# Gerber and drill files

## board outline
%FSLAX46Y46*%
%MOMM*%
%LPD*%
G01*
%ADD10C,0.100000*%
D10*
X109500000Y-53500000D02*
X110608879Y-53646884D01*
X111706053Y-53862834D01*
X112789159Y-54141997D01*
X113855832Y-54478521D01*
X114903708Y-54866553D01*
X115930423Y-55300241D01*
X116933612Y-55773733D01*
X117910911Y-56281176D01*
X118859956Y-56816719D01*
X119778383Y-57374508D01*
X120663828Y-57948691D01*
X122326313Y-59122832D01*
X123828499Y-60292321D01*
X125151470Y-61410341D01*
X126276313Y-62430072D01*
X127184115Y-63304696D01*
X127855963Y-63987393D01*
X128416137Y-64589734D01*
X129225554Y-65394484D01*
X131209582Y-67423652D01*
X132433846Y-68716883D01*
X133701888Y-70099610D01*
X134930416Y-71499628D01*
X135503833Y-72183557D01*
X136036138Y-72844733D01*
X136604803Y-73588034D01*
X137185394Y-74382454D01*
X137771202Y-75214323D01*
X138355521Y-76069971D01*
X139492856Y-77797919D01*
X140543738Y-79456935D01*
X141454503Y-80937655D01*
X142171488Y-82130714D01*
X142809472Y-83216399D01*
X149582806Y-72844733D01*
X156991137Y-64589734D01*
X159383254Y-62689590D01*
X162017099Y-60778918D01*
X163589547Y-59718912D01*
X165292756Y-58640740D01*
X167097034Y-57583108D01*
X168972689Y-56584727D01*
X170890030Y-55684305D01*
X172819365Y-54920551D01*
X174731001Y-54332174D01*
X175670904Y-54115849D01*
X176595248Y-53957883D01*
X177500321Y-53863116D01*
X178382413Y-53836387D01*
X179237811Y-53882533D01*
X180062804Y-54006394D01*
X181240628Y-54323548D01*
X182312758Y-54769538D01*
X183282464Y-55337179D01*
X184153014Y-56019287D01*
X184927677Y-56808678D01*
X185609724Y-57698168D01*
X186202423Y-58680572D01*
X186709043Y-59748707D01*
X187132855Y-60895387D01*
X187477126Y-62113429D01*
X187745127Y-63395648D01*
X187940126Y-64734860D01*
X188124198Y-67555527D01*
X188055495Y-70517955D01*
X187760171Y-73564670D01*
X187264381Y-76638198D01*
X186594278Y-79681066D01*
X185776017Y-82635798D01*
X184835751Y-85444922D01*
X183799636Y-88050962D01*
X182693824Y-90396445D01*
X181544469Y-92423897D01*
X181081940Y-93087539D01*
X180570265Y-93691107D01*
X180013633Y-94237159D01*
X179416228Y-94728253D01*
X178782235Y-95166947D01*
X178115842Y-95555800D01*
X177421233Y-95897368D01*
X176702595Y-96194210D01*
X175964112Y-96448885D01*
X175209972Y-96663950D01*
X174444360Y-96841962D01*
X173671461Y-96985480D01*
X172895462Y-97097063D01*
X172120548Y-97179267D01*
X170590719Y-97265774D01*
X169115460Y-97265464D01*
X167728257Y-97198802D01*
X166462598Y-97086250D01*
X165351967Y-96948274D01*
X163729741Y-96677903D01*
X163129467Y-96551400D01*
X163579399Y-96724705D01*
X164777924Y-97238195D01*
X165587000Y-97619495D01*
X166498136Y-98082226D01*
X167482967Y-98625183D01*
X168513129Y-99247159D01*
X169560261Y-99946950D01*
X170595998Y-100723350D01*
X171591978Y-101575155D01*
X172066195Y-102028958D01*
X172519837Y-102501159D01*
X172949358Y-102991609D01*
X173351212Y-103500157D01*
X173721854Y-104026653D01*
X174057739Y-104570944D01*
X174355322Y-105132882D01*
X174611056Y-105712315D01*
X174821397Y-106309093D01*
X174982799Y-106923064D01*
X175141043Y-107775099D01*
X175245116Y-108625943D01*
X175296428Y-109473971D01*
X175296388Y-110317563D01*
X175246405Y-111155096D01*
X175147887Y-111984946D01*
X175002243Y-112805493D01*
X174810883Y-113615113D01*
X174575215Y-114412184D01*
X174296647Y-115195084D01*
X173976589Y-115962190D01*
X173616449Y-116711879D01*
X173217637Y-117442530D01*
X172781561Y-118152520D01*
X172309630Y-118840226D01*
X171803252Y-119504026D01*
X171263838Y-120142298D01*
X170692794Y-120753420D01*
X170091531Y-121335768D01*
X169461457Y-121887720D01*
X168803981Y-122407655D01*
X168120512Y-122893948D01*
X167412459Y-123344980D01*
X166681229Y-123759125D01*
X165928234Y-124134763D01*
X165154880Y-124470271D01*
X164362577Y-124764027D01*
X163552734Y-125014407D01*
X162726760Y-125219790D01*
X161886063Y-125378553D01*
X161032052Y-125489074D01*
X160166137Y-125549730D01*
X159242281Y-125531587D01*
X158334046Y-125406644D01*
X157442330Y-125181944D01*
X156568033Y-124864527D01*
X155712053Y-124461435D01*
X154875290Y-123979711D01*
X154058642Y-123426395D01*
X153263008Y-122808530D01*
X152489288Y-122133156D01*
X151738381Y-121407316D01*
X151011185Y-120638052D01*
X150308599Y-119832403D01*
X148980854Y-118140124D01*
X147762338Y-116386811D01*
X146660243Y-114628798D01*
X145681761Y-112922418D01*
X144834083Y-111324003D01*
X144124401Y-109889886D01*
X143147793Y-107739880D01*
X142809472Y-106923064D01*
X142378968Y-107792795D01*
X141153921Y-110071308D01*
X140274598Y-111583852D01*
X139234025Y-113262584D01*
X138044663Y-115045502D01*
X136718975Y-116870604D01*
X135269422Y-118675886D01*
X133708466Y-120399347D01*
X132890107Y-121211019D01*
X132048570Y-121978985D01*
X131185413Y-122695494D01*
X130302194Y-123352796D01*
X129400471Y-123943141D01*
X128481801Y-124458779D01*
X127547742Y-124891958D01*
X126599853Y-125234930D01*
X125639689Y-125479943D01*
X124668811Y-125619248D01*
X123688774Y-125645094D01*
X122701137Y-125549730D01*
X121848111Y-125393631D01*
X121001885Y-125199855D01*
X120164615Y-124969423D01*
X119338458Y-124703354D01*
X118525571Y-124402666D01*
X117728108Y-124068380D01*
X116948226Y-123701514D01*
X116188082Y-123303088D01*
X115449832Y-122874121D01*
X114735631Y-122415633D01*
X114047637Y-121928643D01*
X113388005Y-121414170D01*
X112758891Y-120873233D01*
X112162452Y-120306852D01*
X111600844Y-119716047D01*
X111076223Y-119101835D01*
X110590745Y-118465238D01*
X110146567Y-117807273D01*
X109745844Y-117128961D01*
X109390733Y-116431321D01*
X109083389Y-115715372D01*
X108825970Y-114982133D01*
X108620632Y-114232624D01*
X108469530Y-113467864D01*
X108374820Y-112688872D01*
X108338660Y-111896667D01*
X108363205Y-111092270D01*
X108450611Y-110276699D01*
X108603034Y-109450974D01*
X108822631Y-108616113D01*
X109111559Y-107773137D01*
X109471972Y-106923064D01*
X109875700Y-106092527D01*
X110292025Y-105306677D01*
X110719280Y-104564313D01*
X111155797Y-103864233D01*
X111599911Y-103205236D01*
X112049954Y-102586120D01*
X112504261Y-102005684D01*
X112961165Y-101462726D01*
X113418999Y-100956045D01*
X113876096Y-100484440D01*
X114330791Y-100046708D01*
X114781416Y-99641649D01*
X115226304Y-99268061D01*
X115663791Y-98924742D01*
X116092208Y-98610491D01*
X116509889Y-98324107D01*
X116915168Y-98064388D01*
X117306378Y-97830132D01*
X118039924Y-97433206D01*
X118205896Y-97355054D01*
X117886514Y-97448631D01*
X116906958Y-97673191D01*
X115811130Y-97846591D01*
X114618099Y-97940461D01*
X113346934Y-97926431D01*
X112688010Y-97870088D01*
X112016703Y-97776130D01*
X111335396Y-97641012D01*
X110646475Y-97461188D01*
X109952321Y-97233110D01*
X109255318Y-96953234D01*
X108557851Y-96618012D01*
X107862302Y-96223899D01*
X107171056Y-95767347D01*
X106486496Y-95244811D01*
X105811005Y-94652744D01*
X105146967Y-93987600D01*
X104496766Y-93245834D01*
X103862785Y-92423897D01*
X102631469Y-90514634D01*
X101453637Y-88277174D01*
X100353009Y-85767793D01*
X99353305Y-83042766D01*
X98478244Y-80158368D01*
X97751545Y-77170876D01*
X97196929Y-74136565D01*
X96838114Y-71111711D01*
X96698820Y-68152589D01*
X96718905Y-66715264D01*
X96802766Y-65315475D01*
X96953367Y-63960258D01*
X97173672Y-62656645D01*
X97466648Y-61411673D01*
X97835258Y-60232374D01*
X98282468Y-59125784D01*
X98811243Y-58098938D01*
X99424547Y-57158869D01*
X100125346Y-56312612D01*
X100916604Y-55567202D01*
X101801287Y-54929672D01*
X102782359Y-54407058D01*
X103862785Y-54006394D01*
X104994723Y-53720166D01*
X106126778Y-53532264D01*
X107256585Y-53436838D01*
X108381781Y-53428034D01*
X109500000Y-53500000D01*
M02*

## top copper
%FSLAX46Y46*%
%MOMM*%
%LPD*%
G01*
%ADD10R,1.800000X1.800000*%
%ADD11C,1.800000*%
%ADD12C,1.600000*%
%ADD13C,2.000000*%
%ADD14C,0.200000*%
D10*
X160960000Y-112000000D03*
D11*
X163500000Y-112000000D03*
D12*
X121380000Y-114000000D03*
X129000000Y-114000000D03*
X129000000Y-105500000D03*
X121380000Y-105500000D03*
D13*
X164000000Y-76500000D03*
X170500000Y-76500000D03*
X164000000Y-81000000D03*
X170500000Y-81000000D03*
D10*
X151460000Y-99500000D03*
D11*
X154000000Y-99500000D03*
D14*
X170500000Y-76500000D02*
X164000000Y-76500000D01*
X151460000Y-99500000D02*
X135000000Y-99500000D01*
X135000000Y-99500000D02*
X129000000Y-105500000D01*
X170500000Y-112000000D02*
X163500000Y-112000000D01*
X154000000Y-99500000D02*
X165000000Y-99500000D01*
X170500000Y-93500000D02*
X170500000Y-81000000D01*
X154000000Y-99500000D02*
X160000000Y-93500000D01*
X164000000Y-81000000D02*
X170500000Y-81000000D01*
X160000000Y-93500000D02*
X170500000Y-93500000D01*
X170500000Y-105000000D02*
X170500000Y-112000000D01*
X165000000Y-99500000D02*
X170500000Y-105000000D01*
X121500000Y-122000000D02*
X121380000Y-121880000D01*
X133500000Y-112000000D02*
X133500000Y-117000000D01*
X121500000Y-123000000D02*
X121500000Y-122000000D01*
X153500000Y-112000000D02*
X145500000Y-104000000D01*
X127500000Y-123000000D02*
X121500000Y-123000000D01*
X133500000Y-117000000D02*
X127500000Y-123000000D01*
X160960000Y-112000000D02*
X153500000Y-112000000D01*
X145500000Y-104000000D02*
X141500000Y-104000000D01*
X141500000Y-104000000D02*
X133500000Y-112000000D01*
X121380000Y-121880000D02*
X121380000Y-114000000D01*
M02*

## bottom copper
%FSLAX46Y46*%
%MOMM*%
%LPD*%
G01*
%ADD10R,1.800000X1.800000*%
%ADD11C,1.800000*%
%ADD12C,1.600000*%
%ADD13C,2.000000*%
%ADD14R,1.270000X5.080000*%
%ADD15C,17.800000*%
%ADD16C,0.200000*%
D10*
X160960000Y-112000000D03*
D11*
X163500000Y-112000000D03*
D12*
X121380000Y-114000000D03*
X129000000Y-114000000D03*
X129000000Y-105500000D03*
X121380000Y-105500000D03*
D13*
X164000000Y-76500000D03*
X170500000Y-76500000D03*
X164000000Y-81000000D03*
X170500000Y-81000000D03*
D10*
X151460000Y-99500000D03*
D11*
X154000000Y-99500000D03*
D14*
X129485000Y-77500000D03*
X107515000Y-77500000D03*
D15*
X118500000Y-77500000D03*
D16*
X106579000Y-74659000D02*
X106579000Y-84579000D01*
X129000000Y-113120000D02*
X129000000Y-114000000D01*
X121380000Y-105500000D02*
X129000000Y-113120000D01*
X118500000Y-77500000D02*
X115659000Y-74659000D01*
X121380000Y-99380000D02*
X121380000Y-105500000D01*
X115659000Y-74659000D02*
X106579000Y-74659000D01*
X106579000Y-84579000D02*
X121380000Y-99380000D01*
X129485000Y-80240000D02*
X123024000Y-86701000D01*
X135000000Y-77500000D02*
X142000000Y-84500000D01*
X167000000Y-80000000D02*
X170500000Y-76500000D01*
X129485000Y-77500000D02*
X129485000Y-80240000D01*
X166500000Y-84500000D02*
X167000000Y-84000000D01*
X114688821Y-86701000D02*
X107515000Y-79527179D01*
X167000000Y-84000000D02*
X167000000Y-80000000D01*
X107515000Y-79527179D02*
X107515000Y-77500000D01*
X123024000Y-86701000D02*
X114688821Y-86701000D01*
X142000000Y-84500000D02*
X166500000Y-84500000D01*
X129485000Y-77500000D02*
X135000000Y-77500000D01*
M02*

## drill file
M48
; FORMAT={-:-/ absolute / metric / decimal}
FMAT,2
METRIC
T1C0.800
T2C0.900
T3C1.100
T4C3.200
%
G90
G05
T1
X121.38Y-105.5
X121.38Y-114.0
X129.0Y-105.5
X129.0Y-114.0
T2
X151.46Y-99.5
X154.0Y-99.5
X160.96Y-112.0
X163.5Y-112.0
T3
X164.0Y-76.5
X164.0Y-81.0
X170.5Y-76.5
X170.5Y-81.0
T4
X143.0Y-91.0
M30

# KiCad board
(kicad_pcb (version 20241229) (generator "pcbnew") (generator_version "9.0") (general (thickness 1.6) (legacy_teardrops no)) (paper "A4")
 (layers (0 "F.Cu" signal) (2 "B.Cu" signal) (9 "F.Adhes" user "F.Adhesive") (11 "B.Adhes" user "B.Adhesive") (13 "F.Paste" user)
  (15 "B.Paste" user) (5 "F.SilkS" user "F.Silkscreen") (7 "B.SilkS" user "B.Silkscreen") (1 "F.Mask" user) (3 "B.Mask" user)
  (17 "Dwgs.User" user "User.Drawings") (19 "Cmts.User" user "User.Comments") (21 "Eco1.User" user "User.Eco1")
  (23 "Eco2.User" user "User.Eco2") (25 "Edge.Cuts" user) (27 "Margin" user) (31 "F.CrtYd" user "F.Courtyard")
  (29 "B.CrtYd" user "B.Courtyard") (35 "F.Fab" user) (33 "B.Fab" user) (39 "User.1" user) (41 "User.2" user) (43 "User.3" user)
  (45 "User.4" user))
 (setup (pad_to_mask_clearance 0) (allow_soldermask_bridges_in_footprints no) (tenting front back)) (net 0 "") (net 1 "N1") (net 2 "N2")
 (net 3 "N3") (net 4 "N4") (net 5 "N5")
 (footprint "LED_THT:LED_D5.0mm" (layer "F.Cu") (at 160.96 112)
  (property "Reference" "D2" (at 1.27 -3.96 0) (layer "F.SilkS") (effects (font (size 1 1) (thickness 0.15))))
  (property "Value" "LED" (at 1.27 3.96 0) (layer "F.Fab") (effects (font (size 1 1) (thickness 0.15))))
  (pad "1" thru_hole rect (at 0 0) (size 1.8 1.8) (drill 0.9) (layers "*.Cu" "*.Mask") (remove_unused_layers no) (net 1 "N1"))
  (pad "2" thru_hole circle (at 2.54 0) (size 1.8 1.8) (drill 0.9) (layers "*.Cu" "*.Mask") (remove_unused_layers no) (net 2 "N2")))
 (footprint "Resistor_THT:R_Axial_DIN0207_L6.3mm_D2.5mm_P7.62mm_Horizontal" (layer "F.Cu") (at 121.38 114)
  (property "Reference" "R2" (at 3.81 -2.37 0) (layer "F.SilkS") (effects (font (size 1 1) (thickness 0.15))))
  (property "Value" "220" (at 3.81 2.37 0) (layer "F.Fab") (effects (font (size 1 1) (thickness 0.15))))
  (pad "1" thru_hole circle (at 0 0) (size 1.6 1.6) (drill 0.8) (layers "*.Cu" "*.Mask") (remove_unused_layers no) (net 1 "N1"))
  (pad "2" thru_hole circle (at 7.62 0) (size 1.6 1.6) (drill 0.8) (layers "*.Cu" "*.Mask") (remove_unused_layers no) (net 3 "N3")))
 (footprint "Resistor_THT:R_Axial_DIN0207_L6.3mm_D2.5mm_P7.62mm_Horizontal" (layer "F.Cu") (at 129 105.5 180)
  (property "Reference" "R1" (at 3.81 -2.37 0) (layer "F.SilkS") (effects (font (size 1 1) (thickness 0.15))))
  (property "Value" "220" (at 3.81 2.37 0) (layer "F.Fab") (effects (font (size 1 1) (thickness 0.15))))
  (pad "1" thru_hole circle (at 0 0 180) (size 1.6 1.6) (drill 0.8) (layers "*.Cu" "*.Mask") (remove_unused_layers no) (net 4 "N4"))
  (pad "2" thru_hole circle (at 7.62 0 180) (size 1.6 1.6) (drill 0.8) (layers "*.Cu" "*.Mask") (remove_unused_layers no) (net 3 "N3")))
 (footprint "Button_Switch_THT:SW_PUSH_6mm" (layer "F.Cu") (at 164 76.5)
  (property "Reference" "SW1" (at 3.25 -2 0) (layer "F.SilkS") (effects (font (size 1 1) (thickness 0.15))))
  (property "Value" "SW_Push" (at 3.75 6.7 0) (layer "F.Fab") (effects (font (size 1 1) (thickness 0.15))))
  (pad "1" thru_hole circle (at 0 0 90) (size 2 2) (drill 1.1) (layers "*.Cu" "*.Mask") (remove_unused_layers no) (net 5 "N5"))
  (pad "1" thru_hole circle (at 6.5 0 90) (size 2 2) (drill 1.1) (layers "*.Cu" "*.Mask") (remove_unused_layers no) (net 5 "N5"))
  (pad "2" thru_hole circle (at 0 4.5 90) (size 2 2) (drill 1.1) (layers "*.Cu" "*.Mask") (remove_unused_layers no) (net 2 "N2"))
  (pad "2" thru_hole circle (at 6.5 4.5 90) (size 2 2) (drill 1.1) (layers "*.Cu" "*.Mask") (remove_unused_layers no) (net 2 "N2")))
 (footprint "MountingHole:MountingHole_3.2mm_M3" (layer "F.Cu") (at 143 91)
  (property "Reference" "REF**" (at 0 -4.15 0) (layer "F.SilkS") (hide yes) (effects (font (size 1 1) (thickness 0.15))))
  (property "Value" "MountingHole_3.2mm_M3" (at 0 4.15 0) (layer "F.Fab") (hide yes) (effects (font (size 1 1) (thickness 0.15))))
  (pad "" np_thru_hole circle (at 0 0) (size 3.2 3.2) (drill 3.2) (layers "*.Cu" "*.Mask")))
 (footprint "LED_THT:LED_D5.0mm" (layer "F.Cu") (at 151.46 99.5)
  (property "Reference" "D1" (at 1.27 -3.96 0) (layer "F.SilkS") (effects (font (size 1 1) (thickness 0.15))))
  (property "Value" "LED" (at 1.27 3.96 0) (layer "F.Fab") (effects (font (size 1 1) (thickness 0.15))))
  (pad "1" thru_hole rect (at 0 0) (size 1.8 1.8) (drill 0.9) (layers "*.Cu" "*.Mask") (remove_unused_layers no) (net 4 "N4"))
  (pad "2" thru_hole circle (at 2.54 0) (size 1.8 1.8) (drill 0.9) (layers "*.Cu" "*.Mask") (remove_unused_layers no) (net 2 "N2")))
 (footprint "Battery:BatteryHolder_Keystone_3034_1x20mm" (layer "B.Cu") (at 118.5 77.5 180)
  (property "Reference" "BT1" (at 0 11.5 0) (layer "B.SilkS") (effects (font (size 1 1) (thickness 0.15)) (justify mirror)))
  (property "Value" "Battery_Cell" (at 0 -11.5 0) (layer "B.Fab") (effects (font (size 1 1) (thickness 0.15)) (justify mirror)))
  (pad "1" smd rect (at -10.985 0 180) (size 1.27 5.08) (layers "B.Cu" "B.Mask" "B.Paste") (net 5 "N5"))
  (pad "1" smd rect (at 10.985 0 180) (size 1.27 5.08) (layers "B.Cu" "B.Mask" "B.Paste") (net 5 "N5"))
  (pad "2" smd circle (at 0 0 180) (size 17.8 17.8) (layers "B.Cu" "B.Mask") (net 3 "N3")))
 (gr_poly
  (pts (xy 109.5 53.5) (xy 110.608879 53.646884) (xy 111.706053 53.862834) (xy 112.789159 54.141997) (xy 113.855832 54.478521)
   (xy 114.903708 54.866553) (xy 115.930423 55.300241) (xy 116.933612 55.773733) (xy 117.910911 56.281176) (xy 118.859956 56.816719)
   (xy 119.778383 57.374508) (xy 120.663828 57.948691) (xy 122.326313 59.122832) (xy 123.828499 60.292321) (xy 125.15147 61.410341)
   (xy 126.276313 62.430072) (xy 127.184115 63.304696) (xy 127.855963 63.987393) (xy 128.416137 64.589734) (xy 129.225554 65.394484)
   (xy 131.209582 67.423652) (xy 132.433846 68.716883) (xy 133.701888 70.09961) (xy 134.930416 71.499628) (xy 135.503833 72.183557)
   (xy 136.036138 72.844733) (xy 136.604803 73.588034) (xy 137.185394 74.382454) (xy 137.771202 75.214323) (xy 138.355521 76.069971)
   (xy 139.492856 77.797919) (xy 140.543738 79.456935) (xy 141.454503 80.937655) (xy 142.171488 82.130714) (xy 142.809472 83.216399)
   (xy 149.582806 72.844733) (xy 156.991137 64.589734) (xy 159.383254 62.68959) (xy 162.017099 60.778918) (xy 163.589547 59.718912)
   (xy 165.292756 58.64074) (xy 167.097034 57.583108) (xy 168.972689 56.584727) (xy 170.89003 55.684305) (xy 172.819365 54.920551)
   (xy 174.731001 54.332174) (xy 175.670904 54.115849) (xy 176.595248 53.957883) (xy 177.500321 53.863116) (xy 178.382413 53.836387)
   (xy 179.237811 53.882533) (xy 180.062804 54.006394) (xy 181.240628 54.323548) (xy 182.312758 54.769538) (xy 183.282464 55.337179)
   (xy 184.153014 56.019287) (xy 184.927677 56.808678) (xy 185.609724 57.698168) (xy 186.202423 58.680572) (xy 186.709043 59.748707)
   (xy 187.132855 60.895387) (xy 187.477126 62.113429) (xy 187.745127 63.395648) (xy 187.940126 64.73486) (xy 188.124198 67.555527)
   (xy 188.055495 70.517955) (xy 187.760171 73.56467) (xy 187.264381 76.638198) (xy 186.594278 79.681066) (xy 185.776017 82.635798)
   (xy 184.835751 85.444922) (xy 183.799636 88.050962) (xy 182.693824 90.396445) (xy 181.544469 92.423897) (xy 181.08194 93.087539)
   (xy 180.570265 93.691107) (xy 180.013633 94.237159) (xy 179.416228 94.728253) (xy 178.782235 95.166947) (xy 178.115842 95.5558)
   (xy 177.421233 95.897368) (xy 176.702595 96.19421) (xy 175.964112 96.448885) (xy 175.209972 96.66395) (xy 174.44436 96.841962)
   (xy 173.671461 96.98548) (xy 172.895462 97.097063) (xy 172.120548 97.179267) (xy 170.590719 97.265774) (xy 169.11546 97.265464)
   (xy 167.728257 97.198802) (xy 166.462598 97.08625) (xy 165.351967 96.948274) (xy 163.729741 96.677903) (xy 163.129467 96.5514)
   (xy 163.579399 96.724705) (xy 164.777924 97.238195) (xy 165.587 97.619495) (xy 166.498136 98.082226) (xy 167.482967 98.625183)
   (xy 168.513129 99.247159) (xy 169.560261 99.94695) (xy 170.595998 100.72335) (xy 171.591978 101.575155) (xy 172.066195 102.028958)
   (xy 172.519837 102.501159) (xy 172.949358 102.991609) (xy 173.351212 103.500157) (xy 173.721854 104.026653) (xy 174.057739 104.570944)
   (xy 174.355322 105.132882) (xy 174.611056 105.712315) (xy 174.821397 106.309093) (xy 174.982799 106.923064) (xy 175.141043 107.775099)
   (xy 175.245116 108.625943) (xy 175.296428 109.473971) (xy 175.296388 110.317563) (xy 175.246405 111.155096) (xy 175.147887 111.984946)
   (xy 175.002243 112.805493) (xy 174.810883 113.615113) (xy 174.575215 114.412184) (xy 174.296647 115.195084) (xy 173.976589 115.96219)
   (xy 173.616449 116.711879) (xy 173.217637 117.44253) (xy 172.781561 118.15252) (xy 172.30963 118.840226) (xy 171.803252 119.504026)
   (xy 171.263838 120.142298) (xy 170.692794 120.75342) (xy 170.091531 121.335768) (xy 169.461457 121.88772) (xy 168.803981 122.407655)
   (xy 168.120512 122.893948) (xy 167.412459 123.34498) (xy 166.681229 123.759125) (xy 165.928234 124.134763) (xy 165.15488 124.470271)
   (xy 164.362577 124.764027) (xy 163.552734 125.014407) (xy 162.72676 125.21979) (xy 161.886063 125.378553) (xy 161.032052 125.489074)
   (xy 160.166137 125.54973) (xy 159.242281 125.531587) (xy 158.334046 125.406644) (xy 157.44233 125.181944) (xy 156.568033 124.864527)
   (xy 155.712053 124.461435) (xy 154.87529 123.979711) (xy 154.058642 123.426395) (xy 153.263008 122.80853) (xy 152.489288 122.133156)
   (xy 151.738381 121.407316) (xy 151.011185 120.638052) (xy 150.308599 119.832403) (xy 148.980854 118.140124) (xy 147.762338 116.386811)
   (xy 146.660243 114.628798) (xy 145.681761 112.922418) (xy 144.834083 111.324003) (xy 144.124401 109.889886) (xy 143.147793 107.73988)
   (xy 142.809472 106.923064) (xy 142.378968 107.792795) (xy 141.153921 110.071308) (xy 140.274598 111.583852) (xy 139.234025 113.262584)
   (xy 138.044663 115.045502) (xy 136.718975 116.870604) (xy 135.269422 118.675886) (xy 133.708466 120.399347) (xy 132.890107 121.211019)
   (xy 132.04857 121.978985) (xy 131.185413 122.695494) (xy 130.302194 123.352796) (xy 129.400471 123.943141) (xy 128.481801 124.458779)
   (xy 127.547742 124.891958) (xy 126.599853 125.23493) (xy 125.639689 125.479943) (xy 124.668811 125.619248) (xy 123.688774 125.645094)
   (xy 122.701137 125.54973) (xy 121.848111 125.393631) (xy 121.001885 125.199855) (xy 120.164615 124.969423) (xy 119.338458 124.703354)
   (xy 118.525571 124.402666) (xy 117.728108 124.06838) (xy 116.948226 123.701514) (xy 116.188082 123.303088) (xy 115.449832 122.874121)
   (xy 114.735631 122.415633) (xy 114.047637 121.928643) (xy 113.388005 121.41417) (xy 112.758891 120.873233) (xy 112.162452 120.306852)
   (xy 111.600844 119.716047) (xy 111.076223 119.101835) (xy 110.590745 118.465238) (xy 110.146567 117.807273) (xy 109.745844 117.128961)
   (xy 109.390733 116.431321) (xy 109.083389 115.715372) (xy 108.82597 114.982133) (xy 108.620632 114.232624) (xy 108.46953 113.467864)
   (xy 108.37482 112.688872) (xy 108.33866 111.896667) (xy 108.363205 111.09227) (xy 108.450611 110.276699) (xy 108.603034 109.450974)
   (xy 108.822631 108.616113) (xy 109.111559 107.773137) (xy 109.471972 106.923064) (xy 109.8757 106.092527) (xy 110.292025 105.306677)
   (xy 110.71928 104.564313) (xy 111.155797 103.864233) (xy 111.599911 103.205236) (xy 112.049954 102.58612) (xy 112.504261 102.005684)
   (xy 112.961165 101.462726) (xy 113.418999 100.956045) (xy 113.876096 100.48444) (xy 114.330791 100.046708) (xy 114.781416 99.641649)
   (xy 115.226304 99.268061) (xy 115.663791 98.924742) (xy 116.092208 98.610491) (xy 116.509889 98.324107) (xy 116.915168 98.064388)
   (xy 117.306378 97.830132) (xy 118.039924 97.433206) (xy 118.205896 97.355054) (xy 117.886514 97.448631) (xy 116.906958 97.673191)
   (xy 115.81113 97.846591) (xy 114.618099 97.940461) (xy 113.346934 97.926431) (xy 112.68801 97.870088) (xy 112.016703 97.77613)
   (xy 111.335396 97.641012) (xy 110.646475 97.461188) (xy 109.952321 97.23311) (xy 109.255318 96.953234) (xy 108.557851 96.618012)
   (xy 107.862302 96.223899) (xy 107.171056 95.767347) (xy 106.486496 95.244811) (xy 105.811005 94.652744) (xy 105.146967 93.9876)
   (xy 104.496766 93.245834) (xy 103.862785 92.423897) (xy 102.631469 90.514634) (xy 101.453637 88.277174) (xy 100.353009 85.767793)
   (xy 99.353305 83.042766) (xy 98.478244 80.158368) (xy 97.751545 77.170876) (xy 97.196929 74.136565) (xy 96.838114 71.111711)
   (xy 96.69882 68.152589) (xy 96.718905 66.715264) (xy 96.802766 65.315475) (xy 96.953367 63.960258) (xy 97.173672 62.656645)
   (xy 97.466648 61.411673) (xy 97.835258 60.232374) (xy 98.282468 59.125784) (xy 98.811243 58.098938) (xy 99.424547 57.158869)
   (xy 100.125346 56.312612) (xy 100.916604 55.567202) (xy 101.801287 54.929672) (xy 102.782359 54.407058) (xy 103.862785 54.006394)
   (xy 104.994723 53.720166) (xy 106.126778 53.532264) (xy 107.256585 53.436838) (xy 108.381781 53.428034))
  (stroke (width 0) (type solid)) (fill no) (layer "Edge.Cuts"))
 (segment (start 106.579 74.659) (end 106.579 84.579) (width 0.2) (layer "B.Cu") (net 3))
 (segment (start 129 113.12) (end 129 114) (width 0.2) (layer "B.Cu") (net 3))
 (segment (start 121.38 105.5) (end 129 113.12) (width 0.2) (layer "B.Cu") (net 3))
 (segment (start 118.5 77.5) (end 115.659 74.659) (width 0.2) (layer "B.Cu") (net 3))
 (segment (start 121.38 99.38) (end 121.38 105.5) (width 0.2) (layer "B.Cu") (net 3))
 (segment (start 115.659 74.659) (end 106.579 74.659) (width 0.2) (layer "B.Cu") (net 3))
 (segment (start 106.579 84.579) (end 121.38 99.38) (width 0.2) (layer "B.Cu") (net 3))
 (segment (start 170.5 76.5) (end 164 76.5) (width 0.2) (layer "F.Cu") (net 5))
 (segment (start 129.485 80.24) (end 123.024 86.701) (width 0.2) (layer "B.Cu") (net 5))
 (segment (start 135 77.5) (end 142 84.5) (width 0.2) (layer "B.Cu") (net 5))
 (segment (start 167 80) (end 170.5 76.5) (width 0.2) (layer "B.Cu") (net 5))
 (segment (start 129.485 77.5) (end 129.485 80.24) (width 0.2) (layer "B.Cu") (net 5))
 (segment (start 166.5 84.5) (end 167 84) (width 0.2) (layer "B.Cu") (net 5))
 (segment (start 114.688821 86.701) (end 107.515 79.527179) (width 0.2) (layer "B.Cu") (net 5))
 (segment (start 167 84) (end 167 80) (width 0.2) (layer "B.Cu") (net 5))
 (segment (start 107.515 79.527179) (end 107.515 77.5) (width 0.2) (layer "B.Cu") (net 5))
 (segment (start 123.024 86.701) (end 114.688821 86.701) (width 0.2) (layer "B.Cu") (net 5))
 (segment (start 142 84.5) (end 166.5 84.5) (width 0.2) (layer "B.Cu") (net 5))
 (segment (start 129.485 77.5) (end 135 77.5) (width 0.2) (layer "B.Cu") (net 5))
 (segment (start 151.46 99.5) (end 135 99.5) (width 0.2) (layer "F.Cu") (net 4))
 (segment (start 135 99.5) (end 129 105.5) (width 0.2) (layer "F.Cu") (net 4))
 (segment (start 170.5 112) (end 163.5 112) (width 0.2) (layer "F.Cu") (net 2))
 (segment (start 154 99.5) (end 165 99.5) (width 0.2) (layer "F.Cu") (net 2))
 (segment (start 170.5 93.5) (end 170.5 81) (width 0.2) (layer "F.Cu") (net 2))
 (segment (start 154 99.5) (end 160 93.5) (width 0.2) (layer "F.Cu") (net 2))
 (segment (start 164 81) (end 170.5 81) (width 0.2) (layer "F.Cu") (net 2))
 (segment (start 160 93.5) (end 170.5 93.5) (width 0.2) (layer "F.Cu") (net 2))
 (segment (start 170.5 105) (end 170.5 112) (width 0.2) (layer "F.Cu") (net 2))
 (segment (start 165 99.5) (end 170.5 105) (width 0.2) (layer "F.Cu") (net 2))
 (segment (start 121.5 122) (end 121.38 121.88) (width 0.2) (layer "F.Cu") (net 1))
 (segment (start 133.5 112) (end 133.5 117) (width 0.2) (layer "F.Cu") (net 1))
 (segment (start 121.5 123) (end 121.5 122) (width 0.2) (layer "F.Cu") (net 1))
 (segment (start 153.5 112) (end 145.5 104) (width 0.2) (layer "F.Cu") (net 1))
 (segment (start 127.5 123) (end 121.5 123) (width 0.2) (layer "F.Cu") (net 1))
 (segment (start 133.5 117) (end 127.5 123) (width 0.2) (layer "F.Cu") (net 1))
 (segment (start 160.96 112) (end 153.5 112) (width 0.2) (layer "F.Cu") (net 1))
 (segment (start 145.5 104) (end 141.5 104) (width 0.2) (layer "F.Cu") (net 1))
 (segment (start 141.5 104) (end 133.5 112) (width 0.2) (layer "F.Cu") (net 1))
 (segment (start 121.38 121.88) (end 121.38 114) (width 0.2) (layer "F.Cu") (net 1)))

